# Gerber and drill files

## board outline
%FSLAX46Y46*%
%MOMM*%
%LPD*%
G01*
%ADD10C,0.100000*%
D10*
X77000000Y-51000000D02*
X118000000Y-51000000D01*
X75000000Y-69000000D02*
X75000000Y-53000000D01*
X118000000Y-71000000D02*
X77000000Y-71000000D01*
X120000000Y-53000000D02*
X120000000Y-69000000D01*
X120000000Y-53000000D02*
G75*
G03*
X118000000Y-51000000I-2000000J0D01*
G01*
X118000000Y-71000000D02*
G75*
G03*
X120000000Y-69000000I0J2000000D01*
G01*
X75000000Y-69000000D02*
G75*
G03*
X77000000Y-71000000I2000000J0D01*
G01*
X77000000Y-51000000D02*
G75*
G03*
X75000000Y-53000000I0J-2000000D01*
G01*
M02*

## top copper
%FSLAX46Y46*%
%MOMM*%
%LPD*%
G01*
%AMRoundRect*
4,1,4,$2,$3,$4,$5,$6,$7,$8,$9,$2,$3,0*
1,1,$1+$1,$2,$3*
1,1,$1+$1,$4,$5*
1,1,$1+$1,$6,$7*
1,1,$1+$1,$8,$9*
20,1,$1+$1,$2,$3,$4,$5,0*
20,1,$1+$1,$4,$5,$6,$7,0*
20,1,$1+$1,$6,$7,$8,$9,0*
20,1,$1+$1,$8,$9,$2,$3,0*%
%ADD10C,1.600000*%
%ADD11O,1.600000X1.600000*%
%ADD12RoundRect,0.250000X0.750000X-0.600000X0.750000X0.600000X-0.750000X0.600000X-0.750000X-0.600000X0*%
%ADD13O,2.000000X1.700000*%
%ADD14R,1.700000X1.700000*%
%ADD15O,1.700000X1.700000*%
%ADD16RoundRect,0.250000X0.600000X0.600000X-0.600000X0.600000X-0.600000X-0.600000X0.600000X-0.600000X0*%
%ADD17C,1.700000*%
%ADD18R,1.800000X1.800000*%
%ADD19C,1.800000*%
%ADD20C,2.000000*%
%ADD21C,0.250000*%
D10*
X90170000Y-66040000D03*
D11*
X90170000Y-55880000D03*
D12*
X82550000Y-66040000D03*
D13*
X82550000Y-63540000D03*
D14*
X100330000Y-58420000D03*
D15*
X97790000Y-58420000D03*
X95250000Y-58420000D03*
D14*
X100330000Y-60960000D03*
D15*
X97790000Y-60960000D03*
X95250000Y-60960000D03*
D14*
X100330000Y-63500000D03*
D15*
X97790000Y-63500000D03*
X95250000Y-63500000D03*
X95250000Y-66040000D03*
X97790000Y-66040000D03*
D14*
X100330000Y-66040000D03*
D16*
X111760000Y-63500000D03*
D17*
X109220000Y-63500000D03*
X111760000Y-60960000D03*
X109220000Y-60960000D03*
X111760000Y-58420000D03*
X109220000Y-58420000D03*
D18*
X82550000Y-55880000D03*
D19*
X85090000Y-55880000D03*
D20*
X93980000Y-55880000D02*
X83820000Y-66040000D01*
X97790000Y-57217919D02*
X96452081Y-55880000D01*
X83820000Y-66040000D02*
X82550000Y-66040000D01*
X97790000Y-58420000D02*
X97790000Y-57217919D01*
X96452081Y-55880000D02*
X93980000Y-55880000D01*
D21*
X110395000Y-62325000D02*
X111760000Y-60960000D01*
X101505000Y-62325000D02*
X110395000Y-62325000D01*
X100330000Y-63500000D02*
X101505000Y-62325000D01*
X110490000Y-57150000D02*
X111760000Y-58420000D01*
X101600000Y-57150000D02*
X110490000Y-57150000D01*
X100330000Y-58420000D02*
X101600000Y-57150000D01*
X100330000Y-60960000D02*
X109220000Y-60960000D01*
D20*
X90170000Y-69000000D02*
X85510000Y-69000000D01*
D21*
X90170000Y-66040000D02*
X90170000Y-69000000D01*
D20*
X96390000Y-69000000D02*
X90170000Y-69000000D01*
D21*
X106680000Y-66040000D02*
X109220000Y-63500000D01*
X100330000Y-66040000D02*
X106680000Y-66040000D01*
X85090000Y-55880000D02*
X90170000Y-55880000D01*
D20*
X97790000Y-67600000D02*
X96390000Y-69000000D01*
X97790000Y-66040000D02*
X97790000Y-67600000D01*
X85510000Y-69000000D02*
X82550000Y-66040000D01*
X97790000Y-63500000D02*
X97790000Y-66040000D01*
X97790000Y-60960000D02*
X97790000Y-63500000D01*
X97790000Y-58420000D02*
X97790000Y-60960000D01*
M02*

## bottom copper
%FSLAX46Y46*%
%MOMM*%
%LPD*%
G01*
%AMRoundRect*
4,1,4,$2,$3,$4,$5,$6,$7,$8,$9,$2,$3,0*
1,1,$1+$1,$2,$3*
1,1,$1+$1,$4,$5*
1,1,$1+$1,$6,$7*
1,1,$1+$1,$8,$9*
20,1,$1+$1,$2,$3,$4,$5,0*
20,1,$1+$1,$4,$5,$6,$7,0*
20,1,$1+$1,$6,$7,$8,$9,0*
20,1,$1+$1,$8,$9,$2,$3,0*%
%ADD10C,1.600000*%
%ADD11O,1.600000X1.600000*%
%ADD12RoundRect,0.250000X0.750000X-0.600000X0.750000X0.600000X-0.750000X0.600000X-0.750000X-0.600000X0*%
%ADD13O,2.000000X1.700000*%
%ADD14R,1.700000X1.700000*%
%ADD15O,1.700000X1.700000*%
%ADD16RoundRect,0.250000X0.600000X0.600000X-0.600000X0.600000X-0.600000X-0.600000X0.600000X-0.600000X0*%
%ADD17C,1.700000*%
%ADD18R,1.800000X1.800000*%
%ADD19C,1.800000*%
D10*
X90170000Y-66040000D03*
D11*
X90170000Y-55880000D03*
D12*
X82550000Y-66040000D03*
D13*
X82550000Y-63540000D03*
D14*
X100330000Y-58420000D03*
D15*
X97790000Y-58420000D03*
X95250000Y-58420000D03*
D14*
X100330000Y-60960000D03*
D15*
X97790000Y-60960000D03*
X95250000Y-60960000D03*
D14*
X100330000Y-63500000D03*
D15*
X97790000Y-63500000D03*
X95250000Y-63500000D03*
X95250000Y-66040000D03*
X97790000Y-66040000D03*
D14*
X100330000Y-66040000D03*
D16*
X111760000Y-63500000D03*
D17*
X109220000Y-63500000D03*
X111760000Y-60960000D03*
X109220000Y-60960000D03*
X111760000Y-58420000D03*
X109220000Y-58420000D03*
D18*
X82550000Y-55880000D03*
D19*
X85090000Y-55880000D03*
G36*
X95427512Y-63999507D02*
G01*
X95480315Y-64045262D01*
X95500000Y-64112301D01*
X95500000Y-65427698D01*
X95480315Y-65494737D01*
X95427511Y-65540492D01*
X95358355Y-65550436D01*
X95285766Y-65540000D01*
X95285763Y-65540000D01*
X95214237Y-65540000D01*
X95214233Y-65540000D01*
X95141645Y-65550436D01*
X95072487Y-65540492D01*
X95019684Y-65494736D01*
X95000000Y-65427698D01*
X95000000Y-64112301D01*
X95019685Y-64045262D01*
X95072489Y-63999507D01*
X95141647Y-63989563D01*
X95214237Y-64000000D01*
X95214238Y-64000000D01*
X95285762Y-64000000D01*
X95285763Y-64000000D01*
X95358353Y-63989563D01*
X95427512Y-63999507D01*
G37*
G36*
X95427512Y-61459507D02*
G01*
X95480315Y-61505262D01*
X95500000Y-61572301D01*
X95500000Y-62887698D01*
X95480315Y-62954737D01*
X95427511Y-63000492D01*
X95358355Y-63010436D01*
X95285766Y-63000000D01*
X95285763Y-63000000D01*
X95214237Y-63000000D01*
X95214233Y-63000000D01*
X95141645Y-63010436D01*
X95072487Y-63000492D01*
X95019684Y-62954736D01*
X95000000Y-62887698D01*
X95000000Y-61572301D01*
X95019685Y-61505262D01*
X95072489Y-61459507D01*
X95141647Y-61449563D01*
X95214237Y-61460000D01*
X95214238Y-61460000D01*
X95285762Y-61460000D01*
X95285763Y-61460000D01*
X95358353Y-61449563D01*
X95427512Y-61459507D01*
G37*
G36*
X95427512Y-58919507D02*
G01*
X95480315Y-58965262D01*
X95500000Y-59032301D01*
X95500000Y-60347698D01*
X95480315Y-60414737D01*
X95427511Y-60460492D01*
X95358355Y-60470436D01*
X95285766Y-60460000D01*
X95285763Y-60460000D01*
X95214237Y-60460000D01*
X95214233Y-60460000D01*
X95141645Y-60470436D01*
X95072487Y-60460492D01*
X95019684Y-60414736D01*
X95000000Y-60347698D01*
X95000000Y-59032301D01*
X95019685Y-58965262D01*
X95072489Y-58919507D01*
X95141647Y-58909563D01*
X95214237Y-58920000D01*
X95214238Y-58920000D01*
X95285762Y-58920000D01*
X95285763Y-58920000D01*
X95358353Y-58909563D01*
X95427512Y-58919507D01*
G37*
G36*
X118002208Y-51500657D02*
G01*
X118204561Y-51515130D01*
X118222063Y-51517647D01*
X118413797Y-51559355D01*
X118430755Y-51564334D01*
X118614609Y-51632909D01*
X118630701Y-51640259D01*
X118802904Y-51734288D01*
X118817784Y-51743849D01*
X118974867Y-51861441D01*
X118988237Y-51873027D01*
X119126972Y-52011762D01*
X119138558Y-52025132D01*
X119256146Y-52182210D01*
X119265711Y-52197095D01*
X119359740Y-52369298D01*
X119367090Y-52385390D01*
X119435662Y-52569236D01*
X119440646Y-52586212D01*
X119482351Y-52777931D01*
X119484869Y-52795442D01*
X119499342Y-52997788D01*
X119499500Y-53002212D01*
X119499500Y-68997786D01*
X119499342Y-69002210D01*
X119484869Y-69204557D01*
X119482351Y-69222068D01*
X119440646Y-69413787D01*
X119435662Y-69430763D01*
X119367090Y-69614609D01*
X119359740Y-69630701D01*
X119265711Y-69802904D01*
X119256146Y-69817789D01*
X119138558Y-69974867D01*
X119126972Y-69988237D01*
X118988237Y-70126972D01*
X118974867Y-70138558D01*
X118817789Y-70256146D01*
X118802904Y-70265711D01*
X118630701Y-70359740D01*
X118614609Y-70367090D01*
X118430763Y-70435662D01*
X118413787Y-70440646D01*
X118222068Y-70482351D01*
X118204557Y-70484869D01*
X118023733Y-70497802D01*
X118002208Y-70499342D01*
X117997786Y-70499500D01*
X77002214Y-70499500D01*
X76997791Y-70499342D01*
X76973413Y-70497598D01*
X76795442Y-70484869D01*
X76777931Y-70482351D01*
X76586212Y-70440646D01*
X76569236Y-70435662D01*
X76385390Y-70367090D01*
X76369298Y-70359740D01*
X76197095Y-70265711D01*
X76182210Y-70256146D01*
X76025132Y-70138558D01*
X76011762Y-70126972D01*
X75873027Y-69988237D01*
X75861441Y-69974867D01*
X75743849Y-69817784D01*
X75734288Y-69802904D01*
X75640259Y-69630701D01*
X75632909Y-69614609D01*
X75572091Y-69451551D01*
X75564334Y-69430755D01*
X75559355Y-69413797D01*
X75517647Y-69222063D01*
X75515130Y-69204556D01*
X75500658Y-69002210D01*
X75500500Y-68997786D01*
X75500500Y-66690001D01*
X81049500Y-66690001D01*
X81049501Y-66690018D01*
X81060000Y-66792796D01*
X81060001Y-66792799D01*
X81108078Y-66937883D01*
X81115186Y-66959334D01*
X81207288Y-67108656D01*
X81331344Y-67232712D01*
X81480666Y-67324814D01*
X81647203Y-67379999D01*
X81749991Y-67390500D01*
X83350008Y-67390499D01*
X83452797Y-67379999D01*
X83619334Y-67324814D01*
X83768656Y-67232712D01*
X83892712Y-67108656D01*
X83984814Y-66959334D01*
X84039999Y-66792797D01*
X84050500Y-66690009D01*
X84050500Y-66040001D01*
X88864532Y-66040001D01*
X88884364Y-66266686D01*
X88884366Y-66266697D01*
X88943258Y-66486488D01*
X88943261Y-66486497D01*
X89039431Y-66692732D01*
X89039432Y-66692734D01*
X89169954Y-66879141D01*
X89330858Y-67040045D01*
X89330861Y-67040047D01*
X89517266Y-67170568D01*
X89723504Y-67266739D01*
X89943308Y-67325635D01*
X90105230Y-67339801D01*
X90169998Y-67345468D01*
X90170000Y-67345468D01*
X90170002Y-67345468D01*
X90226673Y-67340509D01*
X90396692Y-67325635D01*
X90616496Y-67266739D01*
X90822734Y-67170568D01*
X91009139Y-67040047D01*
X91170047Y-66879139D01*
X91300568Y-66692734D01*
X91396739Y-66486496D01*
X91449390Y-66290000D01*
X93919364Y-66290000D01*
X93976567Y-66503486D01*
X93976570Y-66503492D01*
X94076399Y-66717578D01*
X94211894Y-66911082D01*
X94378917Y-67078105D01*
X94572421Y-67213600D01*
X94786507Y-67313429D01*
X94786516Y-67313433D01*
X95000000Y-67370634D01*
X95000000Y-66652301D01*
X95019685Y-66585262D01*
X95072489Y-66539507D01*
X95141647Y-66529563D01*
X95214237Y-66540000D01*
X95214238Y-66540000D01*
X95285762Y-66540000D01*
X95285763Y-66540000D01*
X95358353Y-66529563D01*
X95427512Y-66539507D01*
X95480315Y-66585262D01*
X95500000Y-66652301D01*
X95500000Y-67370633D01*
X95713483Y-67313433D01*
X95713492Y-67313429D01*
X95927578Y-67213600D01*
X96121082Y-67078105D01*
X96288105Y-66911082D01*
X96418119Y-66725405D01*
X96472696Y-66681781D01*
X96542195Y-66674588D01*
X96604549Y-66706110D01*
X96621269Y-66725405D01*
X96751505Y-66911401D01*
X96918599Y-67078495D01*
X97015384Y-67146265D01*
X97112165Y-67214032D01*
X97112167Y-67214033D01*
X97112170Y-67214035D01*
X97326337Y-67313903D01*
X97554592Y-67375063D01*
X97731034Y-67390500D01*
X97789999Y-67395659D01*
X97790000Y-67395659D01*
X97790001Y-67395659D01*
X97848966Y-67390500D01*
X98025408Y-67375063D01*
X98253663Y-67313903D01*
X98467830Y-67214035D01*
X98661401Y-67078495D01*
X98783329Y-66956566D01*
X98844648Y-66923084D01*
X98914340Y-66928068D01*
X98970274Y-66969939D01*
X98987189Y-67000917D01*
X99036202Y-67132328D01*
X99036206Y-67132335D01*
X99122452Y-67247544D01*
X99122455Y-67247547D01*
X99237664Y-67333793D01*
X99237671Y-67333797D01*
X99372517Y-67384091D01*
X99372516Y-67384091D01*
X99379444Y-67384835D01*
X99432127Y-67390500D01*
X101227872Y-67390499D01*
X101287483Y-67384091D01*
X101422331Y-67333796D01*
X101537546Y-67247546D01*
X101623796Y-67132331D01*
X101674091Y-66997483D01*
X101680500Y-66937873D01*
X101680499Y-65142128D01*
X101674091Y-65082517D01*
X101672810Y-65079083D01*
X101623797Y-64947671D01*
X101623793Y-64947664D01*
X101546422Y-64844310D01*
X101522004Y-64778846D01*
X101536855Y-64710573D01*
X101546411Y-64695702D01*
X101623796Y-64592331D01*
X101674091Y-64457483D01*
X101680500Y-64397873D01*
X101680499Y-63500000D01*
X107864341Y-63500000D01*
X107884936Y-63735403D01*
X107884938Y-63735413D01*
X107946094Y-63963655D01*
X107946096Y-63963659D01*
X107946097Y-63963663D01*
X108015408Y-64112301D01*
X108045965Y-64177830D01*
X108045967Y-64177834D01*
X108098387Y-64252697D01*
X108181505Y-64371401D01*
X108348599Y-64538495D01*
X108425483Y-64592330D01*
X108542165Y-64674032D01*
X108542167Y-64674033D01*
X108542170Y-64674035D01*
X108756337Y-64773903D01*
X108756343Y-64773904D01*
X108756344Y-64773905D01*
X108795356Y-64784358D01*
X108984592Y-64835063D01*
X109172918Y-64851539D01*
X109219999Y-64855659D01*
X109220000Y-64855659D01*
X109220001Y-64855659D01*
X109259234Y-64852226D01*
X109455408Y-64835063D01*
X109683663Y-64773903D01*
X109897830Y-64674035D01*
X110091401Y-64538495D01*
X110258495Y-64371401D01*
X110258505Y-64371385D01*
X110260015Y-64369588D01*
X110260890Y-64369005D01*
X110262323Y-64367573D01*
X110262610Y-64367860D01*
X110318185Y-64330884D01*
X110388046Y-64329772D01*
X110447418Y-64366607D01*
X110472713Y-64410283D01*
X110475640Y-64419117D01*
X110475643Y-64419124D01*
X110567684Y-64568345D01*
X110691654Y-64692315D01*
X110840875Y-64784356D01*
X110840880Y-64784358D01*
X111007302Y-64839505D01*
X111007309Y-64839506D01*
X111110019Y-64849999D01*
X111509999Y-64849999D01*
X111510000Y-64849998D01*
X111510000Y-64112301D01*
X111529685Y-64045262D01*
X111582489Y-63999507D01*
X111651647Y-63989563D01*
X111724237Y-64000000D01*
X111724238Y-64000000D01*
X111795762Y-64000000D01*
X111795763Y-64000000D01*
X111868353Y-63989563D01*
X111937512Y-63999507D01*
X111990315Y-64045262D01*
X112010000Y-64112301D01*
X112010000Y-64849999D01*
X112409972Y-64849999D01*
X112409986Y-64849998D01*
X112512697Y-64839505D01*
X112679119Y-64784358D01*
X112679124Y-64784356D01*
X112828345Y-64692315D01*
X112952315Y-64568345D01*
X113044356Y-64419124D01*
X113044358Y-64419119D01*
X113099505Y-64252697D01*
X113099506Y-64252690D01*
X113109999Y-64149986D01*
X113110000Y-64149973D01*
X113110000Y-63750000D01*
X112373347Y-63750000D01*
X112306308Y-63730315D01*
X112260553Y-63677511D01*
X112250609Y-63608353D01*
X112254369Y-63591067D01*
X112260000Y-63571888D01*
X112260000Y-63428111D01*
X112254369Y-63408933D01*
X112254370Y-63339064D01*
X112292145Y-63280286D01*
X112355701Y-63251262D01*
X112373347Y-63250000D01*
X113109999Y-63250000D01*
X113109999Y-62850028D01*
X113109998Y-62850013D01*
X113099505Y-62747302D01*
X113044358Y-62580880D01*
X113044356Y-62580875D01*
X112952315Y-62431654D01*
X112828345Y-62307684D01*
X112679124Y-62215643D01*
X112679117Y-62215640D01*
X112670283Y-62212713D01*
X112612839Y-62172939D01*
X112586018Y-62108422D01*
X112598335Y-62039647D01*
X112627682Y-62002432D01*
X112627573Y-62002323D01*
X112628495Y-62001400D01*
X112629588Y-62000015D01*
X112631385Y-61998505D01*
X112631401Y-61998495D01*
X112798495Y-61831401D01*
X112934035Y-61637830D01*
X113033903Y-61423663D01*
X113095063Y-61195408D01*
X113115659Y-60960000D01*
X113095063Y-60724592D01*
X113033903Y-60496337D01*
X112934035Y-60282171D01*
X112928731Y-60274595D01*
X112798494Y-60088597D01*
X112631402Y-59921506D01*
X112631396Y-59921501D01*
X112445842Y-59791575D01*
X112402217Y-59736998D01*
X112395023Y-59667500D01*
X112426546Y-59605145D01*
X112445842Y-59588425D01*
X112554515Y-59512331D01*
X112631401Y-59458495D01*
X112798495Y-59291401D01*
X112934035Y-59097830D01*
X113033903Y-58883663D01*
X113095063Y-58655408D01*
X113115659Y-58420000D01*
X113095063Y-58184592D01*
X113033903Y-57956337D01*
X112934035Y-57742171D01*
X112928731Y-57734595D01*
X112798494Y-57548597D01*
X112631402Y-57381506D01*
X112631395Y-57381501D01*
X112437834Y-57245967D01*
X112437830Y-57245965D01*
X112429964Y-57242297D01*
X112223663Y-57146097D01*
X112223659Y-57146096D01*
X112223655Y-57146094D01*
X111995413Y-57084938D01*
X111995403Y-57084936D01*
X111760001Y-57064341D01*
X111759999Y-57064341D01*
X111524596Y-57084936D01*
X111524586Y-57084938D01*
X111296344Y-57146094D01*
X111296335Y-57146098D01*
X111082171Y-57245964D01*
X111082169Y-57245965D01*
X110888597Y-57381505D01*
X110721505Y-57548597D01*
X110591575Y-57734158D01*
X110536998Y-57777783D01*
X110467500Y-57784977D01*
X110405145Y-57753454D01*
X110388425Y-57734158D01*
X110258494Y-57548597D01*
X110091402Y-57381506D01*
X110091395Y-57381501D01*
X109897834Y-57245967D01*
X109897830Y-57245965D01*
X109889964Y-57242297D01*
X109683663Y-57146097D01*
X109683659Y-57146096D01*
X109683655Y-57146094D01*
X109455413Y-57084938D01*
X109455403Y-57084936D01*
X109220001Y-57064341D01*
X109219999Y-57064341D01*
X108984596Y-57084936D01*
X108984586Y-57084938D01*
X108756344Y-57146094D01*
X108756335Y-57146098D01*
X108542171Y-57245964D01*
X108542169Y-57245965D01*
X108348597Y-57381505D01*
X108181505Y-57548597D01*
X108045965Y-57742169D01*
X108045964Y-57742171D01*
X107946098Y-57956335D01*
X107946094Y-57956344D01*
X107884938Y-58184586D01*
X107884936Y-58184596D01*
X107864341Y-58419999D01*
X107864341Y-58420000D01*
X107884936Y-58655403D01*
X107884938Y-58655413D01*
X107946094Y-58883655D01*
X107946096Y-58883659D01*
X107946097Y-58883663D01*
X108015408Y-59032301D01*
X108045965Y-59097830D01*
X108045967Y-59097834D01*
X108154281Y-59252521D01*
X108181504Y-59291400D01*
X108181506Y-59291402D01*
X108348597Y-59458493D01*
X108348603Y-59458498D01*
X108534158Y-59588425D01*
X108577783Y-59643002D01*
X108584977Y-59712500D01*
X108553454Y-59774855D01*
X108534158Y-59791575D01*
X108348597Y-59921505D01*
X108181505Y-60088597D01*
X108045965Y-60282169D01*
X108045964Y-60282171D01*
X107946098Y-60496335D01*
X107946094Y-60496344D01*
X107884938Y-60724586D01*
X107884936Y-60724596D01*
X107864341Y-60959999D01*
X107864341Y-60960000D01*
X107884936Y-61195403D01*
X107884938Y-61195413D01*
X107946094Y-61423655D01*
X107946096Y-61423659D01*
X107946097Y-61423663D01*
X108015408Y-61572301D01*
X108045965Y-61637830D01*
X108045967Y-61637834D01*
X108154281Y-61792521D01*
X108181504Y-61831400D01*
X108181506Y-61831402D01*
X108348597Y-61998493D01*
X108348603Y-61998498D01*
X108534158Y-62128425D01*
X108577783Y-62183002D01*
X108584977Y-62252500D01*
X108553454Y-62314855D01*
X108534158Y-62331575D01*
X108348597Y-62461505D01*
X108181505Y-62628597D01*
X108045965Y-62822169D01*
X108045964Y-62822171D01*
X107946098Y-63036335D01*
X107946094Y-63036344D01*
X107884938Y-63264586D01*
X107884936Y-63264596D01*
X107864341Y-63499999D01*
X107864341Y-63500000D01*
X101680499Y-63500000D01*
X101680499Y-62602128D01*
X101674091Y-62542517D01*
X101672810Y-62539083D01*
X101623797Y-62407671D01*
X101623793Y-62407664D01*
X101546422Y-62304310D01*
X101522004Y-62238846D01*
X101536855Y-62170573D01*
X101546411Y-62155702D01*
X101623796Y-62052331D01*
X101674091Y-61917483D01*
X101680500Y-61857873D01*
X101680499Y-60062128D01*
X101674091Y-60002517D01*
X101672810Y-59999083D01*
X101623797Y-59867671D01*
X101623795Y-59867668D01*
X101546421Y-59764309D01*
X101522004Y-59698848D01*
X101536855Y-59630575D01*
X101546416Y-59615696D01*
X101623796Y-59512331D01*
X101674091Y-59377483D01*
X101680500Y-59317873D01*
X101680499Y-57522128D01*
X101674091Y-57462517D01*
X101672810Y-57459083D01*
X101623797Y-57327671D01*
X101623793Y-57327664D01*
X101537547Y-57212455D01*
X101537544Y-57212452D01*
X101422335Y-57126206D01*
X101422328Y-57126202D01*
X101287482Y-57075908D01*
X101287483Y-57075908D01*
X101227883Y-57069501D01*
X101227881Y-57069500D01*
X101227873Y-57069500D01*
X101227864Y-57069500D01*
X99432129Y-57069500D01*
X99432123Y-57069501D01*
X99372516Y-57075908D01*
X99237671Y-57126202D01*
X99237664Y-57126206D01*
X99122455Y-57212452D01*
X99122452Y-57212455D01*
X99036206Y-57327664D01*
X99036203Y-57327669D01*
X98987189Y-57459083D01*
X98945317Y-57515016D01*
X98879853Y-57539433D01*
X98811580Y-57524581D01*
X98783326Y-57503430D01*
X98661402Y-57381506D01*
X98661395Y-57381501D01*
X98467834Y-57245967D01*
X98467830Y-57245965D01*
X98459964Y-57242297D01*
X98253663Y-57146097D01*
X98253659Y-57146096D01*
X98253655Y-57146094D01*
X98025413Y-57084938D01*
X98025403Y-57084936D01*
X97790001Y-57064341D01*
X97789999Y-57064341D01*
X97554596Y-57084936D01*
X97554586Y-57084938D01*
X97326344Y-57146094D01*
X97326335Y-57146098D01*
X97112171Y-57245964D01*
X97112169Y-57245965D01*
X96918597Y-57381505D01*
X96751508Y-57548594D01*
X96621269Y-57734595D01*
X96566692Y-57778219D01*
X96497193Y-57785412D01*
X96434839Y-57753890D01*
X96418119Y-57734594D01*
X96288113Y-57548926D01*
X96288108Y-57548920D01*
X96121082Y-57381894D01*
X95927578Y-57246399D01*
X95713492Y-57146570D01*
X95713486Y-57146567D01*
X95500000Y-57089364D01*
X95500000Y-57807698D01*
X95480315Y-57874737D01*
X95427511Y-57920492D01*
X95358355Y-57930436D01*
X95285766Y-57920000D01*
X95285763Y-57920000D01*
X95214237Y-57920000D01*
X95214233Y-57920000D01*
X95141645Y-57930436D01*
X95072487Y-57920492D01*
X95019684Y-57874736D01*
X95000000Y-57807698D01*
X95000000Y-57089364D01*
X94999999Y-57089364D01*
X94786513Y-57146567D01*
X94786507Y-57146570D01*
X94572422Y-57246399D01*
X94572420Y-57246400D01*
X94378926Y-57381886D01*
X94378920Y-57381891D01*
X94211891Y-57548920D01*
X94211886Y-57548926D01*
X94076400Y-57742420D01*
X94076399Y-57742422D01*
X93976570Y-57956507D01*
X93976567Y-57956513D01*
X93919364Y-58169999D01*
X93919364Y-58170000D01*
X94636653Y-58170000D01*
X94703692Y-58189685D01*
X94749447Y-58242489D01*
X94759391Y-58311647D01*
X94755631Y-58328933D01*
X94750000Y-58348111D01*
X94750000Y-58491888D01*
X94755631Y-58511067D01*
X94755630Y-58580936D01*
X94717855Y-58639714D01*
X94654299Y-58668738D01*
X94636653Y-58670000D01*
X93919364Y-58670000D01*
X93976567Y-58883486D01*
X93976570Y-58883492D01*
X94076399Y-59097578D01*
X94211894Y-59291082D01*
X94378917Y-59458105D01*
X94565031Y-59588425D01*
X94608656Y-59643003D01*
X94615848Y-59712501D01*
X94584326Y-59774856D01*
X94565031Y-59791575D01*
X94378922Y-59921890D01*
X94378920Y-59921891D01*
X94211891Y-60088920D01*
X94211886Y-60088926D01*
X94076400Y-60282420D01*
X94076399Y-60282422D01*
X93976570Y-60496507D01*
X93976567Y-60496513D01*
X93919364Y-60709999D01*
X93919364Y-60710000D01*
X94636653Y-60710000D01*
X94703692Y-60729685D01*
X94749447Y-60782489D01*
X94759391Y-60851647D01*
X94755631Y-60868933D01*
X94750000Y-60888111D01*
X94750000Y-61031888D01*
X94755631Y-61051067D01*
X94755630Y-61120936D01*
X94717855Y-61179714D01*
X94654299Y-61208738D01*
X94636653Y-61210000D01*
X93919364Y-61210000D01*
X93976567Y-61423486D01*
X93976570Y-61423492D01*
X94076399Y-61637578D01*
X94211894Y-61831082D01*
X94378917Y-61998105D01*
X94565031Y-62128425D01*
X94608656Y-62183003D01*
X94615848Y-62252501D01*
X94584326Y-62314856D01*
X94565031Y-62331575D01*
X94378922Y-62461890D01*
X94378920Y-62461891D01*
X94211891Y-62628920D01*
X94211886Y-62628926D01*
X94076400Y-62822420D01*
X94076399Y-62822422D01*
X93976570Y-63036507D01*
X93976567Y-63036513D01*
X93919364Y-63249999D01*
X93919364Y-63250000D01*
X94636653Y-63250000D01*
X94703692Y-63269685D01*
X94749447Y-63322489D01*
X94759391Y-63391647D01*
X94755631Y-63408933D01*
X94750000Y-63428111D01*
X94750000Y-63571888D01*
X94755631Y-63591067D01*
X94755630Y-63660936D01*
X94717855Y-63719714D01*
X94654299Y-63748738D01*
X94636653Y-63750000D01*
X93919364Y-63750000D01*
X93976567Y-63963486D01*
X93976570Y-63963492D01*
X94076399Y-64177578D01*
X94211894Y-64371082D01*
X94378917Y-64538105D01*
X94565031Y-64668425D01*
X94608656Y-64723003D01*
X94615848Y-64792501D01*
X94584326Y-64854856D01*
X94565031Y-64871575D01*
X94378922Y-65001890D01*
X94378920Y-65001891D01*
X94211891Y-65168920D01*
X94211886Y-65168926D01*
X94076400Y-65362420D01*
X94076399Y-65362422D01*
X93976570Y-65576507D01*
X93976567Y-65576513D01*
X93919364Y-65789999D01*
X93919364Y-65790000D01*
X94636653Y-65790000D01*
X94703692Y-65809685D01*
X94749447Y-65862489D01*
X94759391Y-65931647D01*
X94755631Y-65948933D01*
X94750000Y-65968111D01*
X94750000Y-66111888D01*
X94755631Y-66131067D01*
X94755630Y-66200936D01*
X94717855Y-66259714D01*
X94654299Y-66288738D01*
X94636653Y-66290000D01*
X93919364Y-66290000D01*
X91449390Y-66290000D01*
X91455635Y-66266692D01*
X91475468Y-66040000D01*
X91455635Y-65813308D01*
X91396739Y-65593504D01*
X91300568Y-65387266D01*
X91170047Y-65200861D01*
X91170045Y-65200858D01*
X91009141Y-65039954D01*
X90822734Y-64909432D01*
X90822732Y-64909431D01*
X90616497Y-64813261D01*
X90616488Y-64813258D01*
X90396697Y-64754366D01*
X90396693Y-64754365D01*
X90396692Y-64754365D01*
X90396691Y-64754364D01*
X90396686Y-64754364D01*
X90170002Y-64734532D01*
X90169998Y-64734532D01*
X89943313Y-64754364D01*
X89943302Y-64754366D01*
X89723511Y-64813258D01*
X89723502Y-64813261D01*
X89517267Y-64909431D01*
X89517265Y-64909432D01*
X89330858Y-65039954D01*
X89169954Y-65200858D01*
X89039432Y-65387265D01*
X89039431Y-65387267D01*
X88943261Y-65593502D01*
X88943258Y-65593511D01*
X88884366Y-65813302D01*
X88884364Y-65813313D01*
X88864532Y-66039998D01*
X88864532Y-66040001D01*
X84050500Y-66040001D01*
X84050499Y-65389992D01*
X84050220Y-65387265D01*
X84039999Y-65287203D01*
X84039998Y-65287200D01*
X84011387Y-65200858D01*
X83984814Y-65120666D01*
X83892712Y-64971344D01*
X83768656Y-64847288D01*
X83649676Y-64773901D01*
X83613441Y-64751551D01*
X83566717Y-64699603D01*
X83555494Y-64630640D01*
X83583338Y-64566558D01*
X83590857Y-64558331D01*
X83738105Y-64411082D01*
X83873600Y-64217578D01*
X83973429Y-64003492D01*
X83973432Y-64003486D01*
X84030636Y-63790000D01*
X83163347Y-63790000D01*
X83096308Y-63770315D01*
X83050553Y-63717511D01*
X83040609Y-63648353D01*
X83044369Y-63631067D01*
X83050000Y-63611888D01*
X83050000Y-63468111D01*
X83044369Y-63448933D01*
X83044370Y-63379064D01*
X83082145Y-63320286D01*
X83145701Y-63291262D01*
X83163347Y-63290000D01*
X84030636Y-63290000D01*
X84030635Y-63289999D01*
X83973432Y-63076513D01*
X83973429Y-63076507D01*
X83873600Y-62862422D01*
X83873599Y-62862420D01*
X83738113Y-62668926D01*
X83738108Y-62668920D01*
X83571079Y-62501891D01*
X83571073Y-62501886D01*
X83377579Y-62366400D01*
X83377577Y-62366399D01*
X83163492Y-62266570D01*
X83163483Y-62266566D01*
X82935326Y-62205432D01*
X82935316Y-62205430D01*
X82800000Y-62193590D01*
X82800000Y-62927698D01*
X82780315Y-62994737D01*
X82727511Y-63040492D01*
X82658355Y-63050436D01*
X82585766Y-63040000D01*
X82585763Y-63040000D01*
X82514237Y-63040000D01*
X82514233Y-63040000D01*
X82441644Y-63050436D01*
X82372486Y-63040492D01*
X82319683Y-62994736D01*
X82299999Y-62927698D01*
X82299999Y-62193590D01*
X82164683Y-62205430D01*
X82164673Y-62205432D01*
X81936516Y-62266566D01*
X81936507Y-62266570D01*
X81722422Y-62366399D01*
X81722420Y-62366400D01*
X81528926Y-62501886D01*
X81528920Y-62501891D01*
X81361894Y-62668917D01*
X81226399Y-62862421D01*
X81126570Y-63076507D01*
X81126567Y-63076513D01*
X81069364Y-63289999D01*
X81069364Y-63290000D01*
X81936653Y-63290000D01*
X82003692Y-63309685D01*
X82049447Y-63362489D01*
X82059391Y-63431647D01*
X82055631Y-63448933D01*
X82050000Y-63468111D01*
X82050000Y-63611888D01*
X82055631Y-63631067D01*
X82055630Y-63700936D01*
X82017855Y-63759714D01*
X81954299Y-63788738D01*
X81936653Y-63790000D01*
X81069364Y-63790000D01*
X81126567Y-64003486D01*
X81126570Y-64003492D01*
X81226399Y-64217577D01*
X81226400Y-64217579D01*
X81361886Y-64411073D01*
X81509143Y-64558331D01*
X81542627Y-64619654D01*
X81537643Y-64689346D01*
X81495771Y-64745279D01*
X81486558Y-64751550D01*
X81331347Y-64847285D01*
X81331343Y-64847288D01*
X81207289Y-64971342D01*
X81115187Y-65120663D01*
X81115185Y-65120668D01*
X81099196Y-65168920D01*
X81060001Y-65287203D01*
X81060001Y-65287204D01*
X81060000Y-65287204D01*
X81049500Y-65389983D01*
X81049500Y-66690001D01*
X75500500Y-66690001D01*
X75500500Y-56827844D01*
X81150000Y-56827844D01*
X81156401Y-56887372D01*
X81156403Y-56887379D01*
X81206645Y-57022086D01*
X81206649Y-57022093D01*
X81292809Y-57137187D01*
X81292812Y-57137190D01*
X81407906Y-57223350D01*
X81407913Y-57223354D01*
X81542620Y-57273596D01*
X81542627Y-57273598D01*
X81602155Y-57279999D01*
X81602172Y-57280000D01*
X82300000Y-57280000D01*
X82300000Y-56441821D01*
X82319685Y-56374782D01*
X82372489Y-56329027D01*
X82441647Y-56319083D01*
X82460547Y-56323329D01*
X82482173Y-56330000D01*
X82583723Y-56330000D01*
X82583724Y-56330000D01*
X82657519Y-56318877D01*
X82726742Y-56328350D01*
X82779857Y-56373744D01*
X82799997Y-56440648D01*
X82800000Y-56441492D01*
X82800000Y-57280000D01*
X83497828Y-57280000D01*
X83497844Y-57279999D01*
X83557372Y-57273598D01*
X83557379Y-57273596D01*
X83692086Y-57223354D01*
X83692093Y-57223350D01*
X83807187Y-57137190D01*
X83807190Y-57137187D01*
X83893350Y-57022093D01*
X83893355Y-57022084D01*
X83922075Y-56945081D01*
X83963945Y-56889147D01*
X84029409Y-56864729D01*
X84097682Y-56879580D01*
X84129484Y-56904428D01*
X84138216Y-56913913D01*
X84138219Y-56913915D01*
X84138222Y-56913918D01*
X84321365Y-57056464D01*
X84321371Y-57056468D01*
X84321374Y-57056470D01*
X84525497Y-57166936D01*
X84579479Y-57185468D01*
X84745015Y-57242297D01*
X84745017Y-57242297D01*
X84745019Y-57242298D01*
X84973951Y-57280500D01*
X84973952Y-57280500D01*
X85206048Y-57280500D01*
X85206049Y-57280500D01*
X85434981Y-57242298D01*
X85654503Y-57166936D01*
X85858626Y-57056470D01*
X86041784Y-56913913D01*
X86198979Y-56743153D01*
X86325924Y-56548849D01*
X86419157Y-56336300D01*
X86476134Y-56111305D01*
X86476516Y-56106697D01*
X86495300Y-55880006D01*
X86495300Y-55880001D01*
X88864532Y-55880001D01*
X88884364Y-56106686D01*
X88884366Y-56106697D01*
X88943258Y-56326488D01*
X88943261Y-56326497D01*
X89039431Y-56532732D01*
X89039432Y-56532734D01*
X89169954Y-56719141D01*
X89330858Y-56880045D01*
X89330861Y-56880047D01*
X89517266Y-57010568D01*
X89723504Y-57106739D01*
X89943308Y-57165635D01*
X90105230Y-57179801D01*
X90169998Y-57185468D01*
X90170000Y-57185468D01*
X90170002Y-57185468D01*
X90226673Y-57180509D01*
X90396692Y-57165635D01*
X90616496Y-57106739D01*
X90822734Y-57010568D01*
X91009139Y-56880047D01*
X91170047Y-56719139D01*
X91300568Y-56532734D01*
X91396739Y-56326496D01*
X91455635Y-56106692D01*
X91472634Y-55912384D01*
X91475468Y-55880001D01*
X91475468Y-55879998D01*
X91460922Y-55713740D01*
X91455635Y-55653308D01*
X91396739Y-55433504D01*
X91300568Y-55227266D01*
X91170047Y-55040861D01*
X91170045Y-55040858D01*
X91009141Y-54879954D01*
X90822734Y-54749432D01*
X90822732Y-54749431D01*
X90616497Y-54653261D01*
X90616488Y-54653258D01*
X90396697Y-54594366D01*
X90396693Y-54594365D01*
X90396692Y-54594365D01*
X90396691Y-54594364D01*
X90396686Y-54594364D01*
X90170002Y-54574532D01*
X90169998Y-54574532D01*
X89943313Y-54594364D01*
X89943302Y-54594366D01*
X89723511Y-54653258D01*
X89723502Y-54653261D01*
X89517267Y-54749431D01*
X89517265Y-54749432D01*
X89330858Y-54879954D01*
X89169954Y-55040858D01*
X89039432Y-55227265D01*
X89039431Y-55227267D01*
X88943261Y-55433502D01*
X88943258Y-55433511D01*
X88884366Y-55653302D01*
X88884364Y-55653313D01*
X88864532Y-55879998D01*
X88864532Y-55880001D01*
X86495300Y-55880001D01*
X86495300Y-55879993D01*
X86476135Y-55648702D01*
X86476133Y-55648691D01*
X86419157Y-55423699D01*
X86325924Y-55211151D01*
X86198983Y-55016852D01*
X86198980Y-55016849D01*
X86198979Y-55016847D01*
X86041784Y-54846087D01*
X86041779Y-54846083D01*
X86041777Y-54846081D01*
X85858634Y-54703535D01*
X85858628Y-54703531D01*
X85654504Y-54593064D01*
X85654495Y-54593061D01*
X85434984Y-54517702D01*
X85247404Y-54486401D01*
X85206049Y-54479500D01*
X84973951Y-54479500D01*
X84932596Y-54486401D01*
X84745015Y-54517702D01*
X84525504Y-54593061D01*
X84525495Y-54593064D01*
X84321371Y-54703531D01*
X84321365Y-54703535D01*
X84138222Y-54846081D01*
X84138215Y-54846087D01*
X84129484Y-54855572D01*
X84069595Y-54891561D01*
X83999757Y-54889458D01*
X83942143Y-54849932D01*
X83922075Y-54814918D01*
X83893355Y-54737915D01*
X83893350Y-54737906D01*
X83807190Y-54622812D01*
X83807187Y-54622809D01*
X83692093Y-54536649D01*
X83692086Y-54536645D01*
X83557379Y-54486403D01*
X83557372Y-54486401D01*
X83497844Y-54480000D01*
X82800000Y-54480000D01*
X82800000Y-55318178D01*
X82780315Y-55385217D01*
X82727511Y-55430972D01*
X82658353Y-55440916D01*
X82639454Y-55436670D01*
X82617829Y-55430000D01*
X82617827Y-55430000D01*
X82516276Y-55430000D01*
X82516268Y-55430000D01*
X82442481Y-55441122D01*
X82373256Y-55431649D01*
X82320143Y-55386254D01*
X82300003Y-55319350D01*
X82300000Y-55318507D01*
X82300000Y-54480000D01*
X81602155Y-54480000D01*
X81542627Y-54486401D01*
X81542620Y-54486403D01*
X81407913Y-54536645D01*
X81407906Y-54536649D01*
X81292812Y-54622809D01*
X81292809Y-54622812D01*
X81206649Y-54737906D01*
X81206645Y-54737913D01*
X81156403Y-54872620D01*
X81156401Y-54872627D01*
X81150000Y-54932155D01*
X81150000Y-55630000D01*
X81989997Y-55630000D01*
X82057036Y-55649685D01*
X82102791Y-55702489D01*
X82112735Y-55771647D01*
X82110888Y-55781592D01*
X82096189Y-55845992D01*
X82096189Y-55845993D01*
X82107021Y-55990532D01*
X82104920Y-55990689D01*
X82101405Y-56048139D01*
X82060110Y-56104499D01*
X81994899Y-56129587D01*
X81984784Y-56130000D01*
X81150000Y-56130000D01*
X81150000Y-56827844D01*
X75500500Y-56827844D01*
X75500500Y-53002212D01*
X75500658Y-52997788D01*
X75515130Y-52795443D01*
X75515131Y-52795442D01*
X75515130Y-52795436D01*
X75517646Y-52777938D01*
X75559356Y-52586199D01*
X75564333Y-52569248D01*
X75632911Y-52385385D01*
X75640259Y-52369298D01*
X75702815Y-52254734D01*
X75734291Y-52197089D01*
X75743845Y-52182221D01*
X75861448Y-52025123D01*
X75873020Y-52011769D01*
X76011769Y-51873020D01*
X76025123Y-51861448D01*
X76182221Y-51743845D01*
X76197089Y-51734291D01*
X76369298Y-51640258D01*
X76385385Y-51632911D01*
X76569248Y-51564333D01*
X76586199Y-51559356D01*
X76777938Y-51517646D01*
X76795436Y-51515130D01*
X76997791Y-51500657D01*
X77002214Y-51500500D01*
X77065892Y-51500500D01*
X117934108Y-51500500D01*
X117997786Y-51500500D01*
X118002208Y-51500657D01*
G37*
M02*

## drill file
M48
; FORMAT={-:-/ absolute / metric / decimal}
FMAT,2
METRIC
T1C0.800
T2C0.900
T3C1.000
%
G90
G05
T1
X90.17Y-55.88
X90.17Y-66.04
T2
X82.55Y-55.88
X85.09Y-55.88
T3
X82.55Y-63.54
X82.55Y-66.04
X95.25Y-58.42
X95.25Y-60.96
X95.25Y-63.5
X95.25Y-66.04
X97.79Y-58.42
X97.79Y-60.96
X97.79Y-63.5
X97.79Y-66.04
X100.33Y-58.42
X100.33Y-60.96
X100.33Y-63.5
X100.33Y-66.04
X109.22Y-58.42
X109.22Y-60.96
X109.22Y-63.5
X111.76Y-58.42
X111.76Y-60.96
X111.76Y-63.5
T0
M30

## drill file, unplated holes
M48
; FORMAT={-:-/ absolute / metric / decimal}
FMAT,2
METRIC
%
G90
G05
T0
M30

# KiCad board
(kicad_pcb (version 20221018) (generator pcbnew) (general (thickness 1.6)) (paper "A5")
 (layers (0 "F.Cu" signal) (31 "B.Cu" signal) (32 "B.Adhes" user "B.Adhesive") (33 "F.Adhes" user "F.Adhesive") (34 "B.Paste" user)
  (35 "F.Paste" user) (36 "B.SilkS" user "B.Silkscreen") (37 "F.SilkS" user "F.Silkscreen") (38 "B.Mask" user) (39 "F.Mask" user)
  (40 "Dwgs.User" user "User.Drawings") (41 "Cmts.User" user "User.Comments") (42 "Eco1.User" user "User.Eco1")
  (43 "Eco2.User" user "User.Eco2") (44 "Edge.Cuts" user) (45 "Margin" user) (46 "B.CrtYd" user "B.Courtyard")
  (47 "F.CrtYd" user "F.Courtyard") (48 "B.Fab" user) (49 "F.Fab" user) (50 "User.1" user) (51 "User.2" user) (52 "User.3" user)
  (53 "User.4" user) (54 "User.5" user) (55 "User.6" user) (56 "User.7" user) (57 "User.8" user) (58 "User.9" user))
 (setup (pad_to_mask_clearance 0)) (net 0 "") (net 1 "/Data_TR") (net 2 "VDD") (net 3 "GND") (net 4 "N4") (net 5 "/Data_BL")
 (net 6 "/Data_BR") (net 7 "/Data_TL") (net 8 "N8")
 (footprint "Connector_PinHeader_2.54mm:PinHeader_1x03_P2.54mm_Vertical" (layer "F.Cu") (at 100.33 63.5 -90)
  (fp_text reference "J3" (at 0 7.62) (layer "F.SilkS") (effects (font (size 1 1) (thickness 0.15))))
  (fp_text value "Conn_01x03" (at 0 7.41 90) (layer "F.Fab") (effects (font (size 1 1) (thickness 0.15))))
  (pad "1" thru_hole rect (at 0 0 270) (size 1.7 1.7) (drill 1) (layers "*.Cu" "*.Mask") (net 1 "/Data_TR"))
  (pad "2" thru_hole oval (at 0 2.54 270) (size 1.7 1.7) (drill 1) (layers "*.Cu" "*.Mask") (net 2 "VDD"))
  (pad "3" thru_hole oval (at 0 5.08 270) (size 1.7 1.7) (drill 1) (layers "*.Cu" "*.Mask") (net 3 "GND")))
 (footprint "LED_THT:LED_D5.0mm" (layer "F.Cu") (at 82.55 55.88)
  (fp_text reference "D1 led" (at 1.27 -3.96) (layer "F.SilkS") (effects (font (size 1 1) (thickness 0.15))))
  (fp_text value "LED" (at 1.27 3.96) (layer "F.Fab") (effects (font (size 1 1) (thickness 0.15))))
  (pad "1" thru_hole rect (at 0 0) (size 1.8 1.8) (drill 0.9) (layers "*.Cu" "*.Mask") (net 3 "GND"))
  (pad "2" thru_hole circle (at 2.54 0) (size 1.8 1.8) (drill 0.9) (layers "*.Cu" "*.Mask") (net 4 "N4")))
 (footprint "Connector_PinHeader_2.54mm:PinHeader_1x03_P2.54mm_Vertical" (layer "F.Cu") (at 100.33 58.42 -90)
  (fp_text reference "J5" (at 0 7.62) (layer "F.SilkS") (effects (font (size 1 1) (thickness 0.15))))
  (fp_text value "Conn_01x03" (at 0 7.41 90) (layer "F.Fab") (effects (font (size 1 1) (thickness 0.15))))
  (pad "1" thru_hole rect (at 0 0 270) (size 1.7 1.7) (drill 1) (layers "*.Cu" "*.Mask") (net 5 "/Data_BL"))
  (pad "2" thru_hole oval (at 0 2.54 270) (size 1.7 1.7) (drill 1) (layers "*.Cu" "*.Mask") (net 2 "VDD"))
  (pad "3" thru_hole oval (at 0 5.08 270) (size 1.7 1.7) (drill 1) (layers "*.Cu" "*.Mask") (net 3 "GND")))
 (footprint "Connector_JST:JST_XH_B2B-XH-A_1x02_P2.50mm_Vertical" (layer "F.Cu") (at 82.55 66.04 90)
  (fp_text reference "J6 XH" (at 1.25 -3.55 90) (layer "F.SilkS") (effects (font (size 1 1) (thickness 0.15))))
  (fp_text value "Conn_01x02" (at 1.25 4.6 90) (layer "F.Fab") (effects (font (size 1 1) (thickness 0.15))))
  (pad "1" thru_hole roundrect (at 0 0 90) (size 1.7 2) (drill 1) (layers "*.Cu" "*.Mask") (roundrect_rratio 0.1470588235) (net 2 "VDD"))
  (pad "2" thru_hole oval (at 2.5 0 90) (size 1.7 2) (drill 1) (layers "*.Cu" "*.Mask") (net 3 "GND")))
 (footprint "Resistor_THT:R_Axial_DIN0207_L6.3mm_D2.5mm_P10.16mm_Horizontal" (layer "F.Cu") (at 90.17 66.04 90)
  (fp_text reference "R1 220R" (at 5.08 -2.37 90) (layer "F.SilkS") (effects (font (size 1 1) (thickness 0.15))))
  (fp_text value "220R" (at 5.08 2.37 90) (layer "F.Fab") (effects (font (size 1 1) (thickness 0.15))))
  (pad "1" thru_hole circle (at 0 0 90) (size 1.6 1.6) (drill 0.8) (layers "*.Cu" "*.Mask") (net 2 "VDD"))
  (pad "2" thru_hole oval (at 10.16 0 90) (size 1.6 1.6) (drill 0.8) (layers "*.Cu" "*.Mask") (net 4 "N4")))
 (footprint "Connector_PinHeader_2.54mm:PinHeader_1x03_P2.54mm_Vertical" (layer "F.Cu") (at 100.33 60.96 -90)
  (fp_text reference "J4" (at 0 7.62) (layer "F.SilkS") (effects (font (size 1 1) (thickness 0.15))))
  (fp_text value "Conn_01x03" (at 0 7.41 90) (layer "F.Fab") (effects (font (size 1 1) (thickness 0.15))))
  (pad "1" thru_hole rect (at 0 0 270) (size 1.7 1.7) (drill 1) (layers "*.Cu" "*.Mask") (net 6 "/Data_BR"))
  (pad "2" thru_hole oval (at 0 2.54 270) (size 1.7 1.7) (drill 1) (layers "*.Cu" "*.Mask") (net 2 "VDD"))
  (pad "3" thru_hole oval (at 0 5.08 270) (size 1.7 1.7) (drill 1) (layers "*.Cu" "*.Mask") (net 3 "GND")))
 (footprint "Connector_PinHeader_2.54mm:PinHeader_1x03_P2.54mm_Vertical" (layer "F.Cu") (at 100.33 66.04 -90)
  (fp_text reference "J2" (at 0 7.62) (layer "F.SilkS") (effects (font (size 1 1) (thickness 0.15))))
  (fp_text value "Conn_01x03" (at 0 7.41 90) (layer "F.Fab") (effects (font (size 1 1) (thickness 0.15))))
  (pad "1" thru_hole rect (at 0 0 270) (size 1.7 1.7) (drill 1) (layers "*.Cu" "*.Mask") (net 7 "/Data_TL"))
  (pad "2" thru_hole oval (at 0 2.54 270) (size 1.7 1.7) (drill 1) (layers "*.Cu" "*.Mask") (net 2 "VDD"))
  (pad "3" thru_hole oval (at 0 5.08 270) (size 1.7 1.7) (drill 1) (layers "*.Cu" "*.Mask") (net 3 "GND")))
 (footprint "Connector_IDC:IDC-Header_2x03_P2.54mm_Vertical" (layer "F.Cu") (at 111.76 63.5 180)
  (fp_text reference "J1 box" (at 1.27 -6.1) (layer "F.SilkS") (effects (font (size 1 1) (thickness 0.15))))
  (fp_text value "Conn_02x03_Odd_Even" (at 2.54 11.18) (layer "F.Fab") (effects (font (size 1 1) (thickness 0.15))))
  (pad "1" thru_hole roundrect (at 0 0 180) (size 1.7 1.7) (drill 1) (layers "*.Cu" "*.Mask") (roundrect_rratio 0.1470588235) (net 3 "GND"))
  (pad "2" thru_hole circle (at 2.54 0 180) (size 1.7 1.7) (drill 1) (layers "*.Cu" "*.Mask") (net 7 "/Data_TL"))
  (pad "3" thru_hole circle (at 0 2.54 180) (size 1.7 1.7) (drill 1) (layers "*.Cu" "*.Mask") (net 1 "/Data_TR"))
  (pad "4" thru_hole circle (at 2.54 2.54 180) (size 1.7 1.7) (drill 1) (layers "*.Cu" "*.Mask") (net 6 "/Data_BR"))
  (pad "5" thru_hole circle (at 0 5.08 180) (size 1.7 1.7) (drill 1) (layers "*.Cu" "*.Mask") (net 5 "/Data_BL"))
  (pad "6" thru_hole circle (at 2.54 5.08 180) (size 1.7 1.7) (drill 1) (layers "*.Cu" "*.Mask") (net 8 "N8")))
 (gr_arc (start 77 71) (mid 75.585786 70.414214) (end 75 69) (stroke (width 0.1) (type default)) (layer "Edge.Cuts"))
 (gr_line (start 75 69) (end 75 53) (stroke (width 0.1) (type default)) (layer "Edge.Cuts"))
 (gr_line (start 118 71) (end 77 71) (stroke (width 0.1) (type default)) (layer "Edge.Cuts"))
 (gr_arc (start 75 53) (mid 75.585786 51.585786) (end 77 51) (stroke (width 0.1) (type default)) (layer "Edge.Cuts"))
 (gr_arc (start 120 69) (mid 119.414214 70.414214) (end 118 71) (stroke (width 0.1) (type default)) (layer "Edge.Cuts"))
 (gr_line (start 77 51) (end 118 51) (stroke (width 0.1) (type default)) (layer "Edge.Cuts"))
 (gr_line (start 120 53) (end 120 69) (stroke (width 0.1) (type default)) (layer "Edge.Cuts"))
 (gr_arc (start 118 51) (mid 119.414214 51.585786) (end 120 53) (stroke (width 0.1) (type default)) (layer "Edge.Cuts"))
 (segment (start 85.09 55.88) (end 90.17 55.88) (width 0.25) (layer "F.Cu") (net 4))
 (segment (start 90.17 66.04) (end 90.17 69) (width 0.25) (layer "F.Cu") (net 2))
 (segment (start 96.39 69) (end 90.17 69) (width 2) (layer "F.Cu") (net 2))
 (segment (start 97.79 63.5) (end 97.79 66.04) (width 2) (layer "F.Cu") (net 2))
 (segment (start 97.79 67.6) (end 96.39 69) (width 2) (layer "F.Cu") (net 2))
 (segment (start 97.79 60.96) (end 97.79 63.5) (width 2) (layer "F.Cu") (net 2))
 (segment (start 97.79 66.04) (end 97.79 67.6) (width 2) (layer "F.Cu") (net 2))
 (segment (start 97.79 58.42) (end 97.79 60.96) (width 2) (layer "F.Cu") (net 2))
 (segment (start 93.98 55.88) (end 83.82 66.04) (width 2) (layer "F.Cu") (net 2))
 (segment (start 97.79 58.42) (end 97.79 57.217919) (width 2) (layer "F.Cu") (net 2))
 (segment (start 85.51 69) (end 82.55 66.04) (width 2) (layer "F.Cu") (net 2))
 (segment (start 96.452081 55.88) (end 93.98 55.88) (width 2) (layer "F.Cu") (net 2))
 (segment (start 90.17 69) (end 85.51 69) (width 2) (layer "F.Cu") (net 2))
 (segment (start 83.82 66.04) (end 82.55 66.04) (width 2) (layer "F.Cu") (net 2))
 (segment (start 97.79 57.217919) (end 96.452081 55.88) (width 2) (layer "F.Cu") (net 2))
 (segment (start 100.33 66.04) (end 106.68 66.04) (width 0.25) (layer "F.Cu") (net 7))
 (segment (start 106.68 66.04) (end 109.22 63.5) (width 0.25) (layer "F.Cu") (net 7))
 (segment (start 100.33 63.5) (end 101.505 62.325) (width 0.25) (layer "F.Cu") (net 1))
 (segment (start 110.395 62.325) (end 111.76 60.96) (width 0.25) (layer "F.Cu") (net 1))
 (segment (start 101.505 62.325) (end 110.395 62.325) (width 0.25) (layer "F.Cu") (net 1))
 (segment (start 100.33 60.96) (end 109.22 60.96) (width 0.25) (layer "F.Cu") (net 6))
 (segment (start 101.6 57.15) (end 110.49 57.15) (width 0.25) (layer "F.Cu") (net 5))
 (segment (start 110.49 57.15) (end 111.76 58.42) (width 0.25) (layer "F.Cu") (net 5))
 (segment (start 100.33 58.42) (end 101.6 57.15) (width 0.25) (layer "F.Cu") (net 5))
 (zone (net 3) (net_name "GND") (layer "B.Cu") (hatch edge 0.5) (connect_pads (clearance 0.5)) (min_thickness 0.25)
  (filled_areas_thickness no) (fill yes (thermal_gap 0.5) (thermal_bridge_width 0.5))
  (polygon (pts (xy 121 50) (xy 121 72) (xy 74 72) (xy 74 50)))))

